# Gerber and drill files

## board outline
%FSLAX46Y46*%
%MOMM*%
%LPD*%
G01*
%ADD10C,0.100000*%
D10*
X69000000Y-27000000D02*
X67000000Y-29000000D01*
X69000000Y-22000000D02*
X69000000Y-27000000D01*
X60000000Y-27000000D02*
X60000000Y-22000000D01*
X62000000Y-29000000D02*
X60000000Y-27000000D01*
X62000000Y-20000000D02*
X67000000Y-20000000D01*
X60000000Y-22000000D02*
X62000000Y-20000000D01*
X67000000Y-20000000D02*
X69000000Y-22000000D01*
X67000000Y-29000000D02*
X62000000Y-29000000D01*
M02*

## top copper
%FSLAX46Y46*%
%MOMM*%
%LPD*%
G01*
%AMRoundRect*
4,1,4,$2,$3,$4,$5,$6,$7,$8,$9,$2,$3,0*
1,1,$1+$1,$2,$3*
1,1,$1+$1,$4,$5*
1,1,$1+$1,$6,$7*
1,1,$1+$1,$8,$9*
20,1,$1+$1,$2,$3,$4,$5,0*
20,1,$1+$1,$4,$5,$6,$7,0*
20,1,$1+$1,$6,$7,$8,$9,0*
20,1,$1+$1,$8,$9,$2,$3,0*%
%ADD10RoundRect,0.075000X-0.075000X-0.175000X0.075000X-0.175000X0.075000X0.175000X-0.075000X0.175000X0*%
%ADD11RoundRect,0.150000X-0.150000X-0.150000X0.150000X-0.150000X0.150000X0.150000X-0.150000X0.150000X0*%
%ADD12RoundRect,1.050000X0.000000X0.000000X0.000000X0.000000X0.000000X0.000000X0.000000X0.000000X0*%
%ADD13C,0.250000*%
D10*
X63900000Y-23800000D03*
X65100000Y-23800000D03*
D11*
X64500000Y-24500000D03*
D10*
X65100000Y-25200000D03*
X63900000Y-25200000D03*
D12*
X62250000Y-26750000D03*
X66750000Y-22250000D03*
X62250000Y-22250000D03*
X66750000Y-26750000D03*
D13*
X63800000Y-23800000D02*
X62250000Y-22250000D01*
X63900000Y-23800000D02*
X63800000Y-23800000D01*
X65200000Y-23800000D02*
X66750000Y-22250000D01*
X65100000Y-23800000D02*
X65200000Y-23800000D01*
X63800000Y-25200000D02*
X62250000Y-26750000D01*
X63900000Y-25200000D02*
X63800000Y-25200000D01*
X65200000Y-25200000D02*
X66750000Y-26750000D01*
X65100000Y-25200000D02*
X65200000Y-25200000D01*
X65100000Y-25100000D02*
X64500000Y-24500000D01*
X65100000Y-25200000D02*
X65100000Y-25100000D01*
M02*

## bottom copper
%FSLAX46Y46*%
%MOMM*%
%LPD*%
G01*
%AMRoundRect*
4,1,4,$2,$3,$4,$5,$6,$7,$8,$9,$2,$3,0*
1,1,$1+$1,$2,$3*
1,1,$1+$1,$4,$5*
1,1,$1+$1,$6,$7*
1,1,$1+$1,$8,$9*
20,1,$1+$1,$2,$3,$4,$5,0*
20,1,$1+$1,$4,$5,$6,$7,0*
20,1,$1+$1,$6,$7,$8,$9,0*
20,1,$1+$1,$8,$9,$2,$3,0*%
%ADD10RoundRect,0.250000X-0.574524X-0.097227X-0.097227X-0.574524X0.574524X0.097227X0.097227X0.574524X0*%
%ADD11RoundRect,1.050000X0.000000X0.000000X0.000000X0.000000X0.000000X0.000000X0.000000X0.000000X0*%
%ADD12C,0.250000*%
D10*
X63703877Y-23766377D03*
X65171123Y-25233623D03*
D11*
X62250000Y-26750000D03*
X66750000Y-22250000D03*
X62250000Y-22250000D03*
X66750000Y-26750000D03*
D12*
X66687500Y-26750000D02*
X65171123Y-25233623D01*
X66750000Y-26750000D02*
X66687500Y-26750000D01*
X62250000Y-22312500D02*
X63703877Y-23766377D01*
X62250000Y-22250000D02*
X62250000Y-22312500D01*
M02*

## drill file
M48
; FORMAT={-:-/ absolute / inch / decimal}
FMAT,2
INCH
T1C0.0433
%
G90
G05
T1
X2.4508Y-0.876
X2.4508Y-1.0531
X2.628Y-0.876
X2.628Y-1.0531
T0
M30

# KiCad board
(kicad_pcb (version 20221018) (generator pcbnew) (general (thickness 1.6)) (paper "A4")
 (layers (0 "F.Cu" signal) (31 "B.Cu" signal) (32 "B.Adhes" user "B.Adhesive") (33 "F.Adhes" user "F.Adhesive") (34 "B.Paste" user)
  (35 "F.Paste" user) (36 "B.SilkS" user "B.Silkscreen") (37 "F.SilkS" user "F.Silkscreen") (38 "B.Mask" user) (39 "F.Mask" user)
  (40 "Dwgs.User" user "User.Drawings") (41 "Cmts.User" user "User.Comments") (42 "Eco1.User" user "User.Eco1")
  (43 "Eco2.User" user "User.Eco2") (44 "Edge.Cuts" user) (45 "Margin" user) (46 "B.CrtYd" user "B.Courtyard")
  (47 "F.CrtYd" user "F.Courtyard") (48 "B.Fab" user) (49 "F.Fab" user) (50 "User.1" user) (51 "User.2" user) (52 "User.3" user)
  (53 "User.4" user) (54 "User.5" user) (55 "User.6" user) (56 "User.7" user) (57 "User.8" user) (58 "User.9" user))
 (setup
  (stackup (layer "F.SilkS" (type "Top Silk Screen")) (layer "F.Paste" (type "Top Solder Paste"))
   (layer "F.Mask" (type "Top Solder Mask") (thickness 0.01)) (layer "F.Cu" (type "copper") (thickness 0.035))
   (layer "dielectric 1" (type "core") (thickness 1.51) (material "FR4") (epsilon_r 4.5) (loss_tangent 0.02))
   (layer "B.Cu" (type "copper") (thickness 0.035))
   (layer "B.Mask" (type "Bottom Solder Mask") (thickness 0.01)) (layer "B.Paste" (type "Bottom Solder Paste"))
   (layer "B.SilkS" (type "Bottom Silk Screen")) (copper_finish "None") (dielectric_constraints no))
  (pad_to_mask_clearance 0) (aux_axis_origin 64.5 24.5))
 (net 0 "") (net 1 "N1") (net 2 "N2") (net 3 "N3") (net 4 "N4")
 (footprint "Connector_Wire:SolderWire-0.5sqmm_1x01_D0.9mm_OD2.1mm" (layer "F.Cu") (at 62.25 26.75)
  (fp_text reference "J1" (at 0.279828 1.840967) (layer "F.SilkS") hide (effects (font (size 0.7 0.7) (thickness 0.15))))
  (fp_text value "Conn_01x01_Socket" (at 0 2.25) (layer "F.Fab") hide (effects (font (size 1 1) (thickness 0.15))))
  (pad "1" thru_hole roundrect (at 0 0) (size 2.1 2.1) (drill 1.1) (layers "*.Cu" "*.Mask") (roundrect_rratio 0.5) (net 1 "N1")))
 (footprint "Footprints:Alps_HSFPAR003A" (layer "F.Cu") (at 64.5 24.5)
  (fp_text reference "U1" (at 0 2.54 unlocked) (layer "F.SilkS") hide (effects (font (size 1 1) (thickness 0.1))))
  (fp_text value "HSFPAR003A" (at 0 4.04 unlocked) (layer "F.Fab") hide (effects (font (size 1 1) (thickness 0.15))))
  (pad "1" smd roundrect (at -0.6 -0.7) (size 0.3 0.5) (layers "F.Cu" "F.Paste" "F.Mask") (roundrect_rratio 0.25) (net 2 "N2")
   (thermal_bridge_angle 45))
  (pad "2" smd roundrect (at 0.6 -0.7) (size 0.3 0.5) (layers "F.Cu" "F.Paste" "F.Mask") (roundrect_rratio 0.25) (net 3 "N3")
   (thermal_bridge_angle 45))
  (pad "3" smd roundrect (at 0 0) (size 0.6 0.6) (layers "F.Cu" "F.Paste" "F.Mask") (roundrect_rratio 0.25) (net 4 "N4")
   (thermal_bridge_angle 45))
  (pad "3" smd roundrect (at 0.6 0.7) (size 0.3 0.5) (layers "F.Cu" "F.Paste" "F.Mask") (roundrect_rratio 0.25) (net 4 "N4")
   (thermal_bridge_angle 45))
  (pad "4" smd roundrect (at -0.6 0.7) (size 0.3 0.5) (layers "F.Cu" "F.Paste" "F.Mask") (roundrect_rratio 0.25) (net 1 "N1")
   (thermal_bridge_angle 45)))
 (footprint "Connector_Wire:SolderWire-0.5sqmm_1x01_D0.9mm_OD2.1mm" (layer "F.Cu") (at 66.75 22.25)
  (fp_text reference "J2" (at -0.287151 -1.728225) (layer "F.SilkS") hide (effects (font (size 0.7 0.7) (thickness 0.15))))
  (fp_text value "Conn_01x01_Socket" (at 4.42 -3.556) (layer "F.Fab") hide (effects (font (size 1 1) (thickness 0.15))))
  (pad "1" thru_hole roundrect (at 0 0) (size 2.1 2.1) (drill 1.1) (layers "*.Cu" "*.Mask") (roundrect_rratio 0.5) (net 3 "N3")))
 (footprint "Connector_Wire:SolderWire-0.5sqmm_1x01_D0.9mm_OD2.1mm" (layer "F.Cu") (at 62.25 22.25)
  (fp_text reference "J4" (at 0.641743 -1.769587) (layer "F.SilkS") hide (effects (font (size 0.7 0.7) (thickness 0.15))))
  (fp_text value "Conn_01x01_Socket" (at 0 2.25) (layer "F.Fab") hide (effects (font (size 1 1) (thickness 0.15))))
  (pad "1" thru_hole roundrect (at 0 0) (size 2.1 2.1) (drill 1.1) (layers "*.Cu" "*.Mask") (roundrect_rratio 0.5) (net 2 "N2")))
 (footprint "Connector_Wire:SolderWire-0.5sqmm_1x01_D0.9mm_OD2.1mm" (layer "F.Cu") (at 66.75 26.75)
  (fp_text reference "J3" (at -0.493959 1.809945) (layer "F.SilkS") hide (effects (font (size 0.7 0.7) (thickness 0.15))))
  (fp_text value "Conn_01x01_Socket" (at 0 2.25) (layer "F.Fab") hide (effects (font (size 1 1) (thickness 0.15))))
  (pad "1" thru_hole roundrect (at 0 0) (size 2.1 2.1) (drill 1.1) (layers "*.Cu" "*.Mask") (roundrect_rratio 0.5) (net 4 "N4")
   (clearance -1)))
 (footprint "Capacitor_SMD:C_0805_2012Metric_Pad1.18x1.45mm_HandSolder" (layer "B.Cu") (at 64.4375 24.5 -45)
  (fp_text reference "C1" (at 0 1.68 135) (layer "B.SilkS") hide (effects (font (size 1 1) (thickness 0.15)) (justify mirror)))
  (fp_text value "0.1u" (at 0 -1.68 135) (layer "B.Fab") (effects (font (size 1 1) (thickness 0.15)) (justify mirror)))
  (pad "1" smd roundrect (at -1.0375 0 315) (size 1.175 1.45) (layers "B.Cu" "B.Paste" "B.Mask") (roundrect_rratio 0.2127659574)
   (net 2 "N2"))
  (pad "2" smd roundrect (at 1.0375 0 315) (size 1.175 1.45) (layers "B.Cu" "B.Paste" "B.Mask") (roundrect_rratio 0.2127659574) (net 4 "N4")))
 (gr_line (start 69 27) (end 67 29) (stroke (width 0.1) (type default)) (layer "Edge.Cuts"))
 (gr_line (start 69 22) (end 69 27) (stroke (width 0.1) (type default)) (layer "Edge.Cuts"))
 (gr_line (start 60 27) (end 60 22) (stroke (width 0.1) (type default)) (layer "Edge.Cuts"))
 (gr_line (start 62 29) (end 60 27) (stroke (width 0.1) (type default)) (layer "Edge.Cuts"))
 (gr_line (start 62 20) (end 67 20) (stroke (width 0.1) (type default)) (layer "Edge.Cuts"))
 (gr_line (start 60 22) (end 62 20) (stroke (width 0.1) (type default)) (layer "Edge.Cuts"))
 (gr_line (start 67 20) (end 69 22) (stroke (width 0.1) (type default)) (layer "Edge.Cuts"))
 (gr_line (start 67 29) (end 62 29) (stroke (width 0.1) (type default)) (layer "Edge.Cuts"))
 (segment (start 63.8 23.8) (end 62.25 22.25) (width 0.25) (layer "F.Cu") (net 2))
 (segment (start 63.9 23.8) (end 63.8 23.8) (width 0.25) (layer "F.Cu") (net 2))
 (segment (start 62.25 22.25) (end 62.25 22.3125) (width 0.25) (layer "B.Cu") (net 2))
 (segment (start 62.25 22.3125) (end 63.703877 23.766377) (width 0.25) (layer "B.Cu") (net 2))
 (segment (start 65.2 23.8) (end 66.75 22.25) (width 0.25) (layer "F.Cu") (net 3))
 (segment (start 65.1 23.8) (end 65.2 23.8) (width 0.25) (layer "F.Cu") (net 3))
 (segment (start 65.1 25.1) (end 64.5 24.5) (width 0.25) (layer "F.Cu") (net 4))
 (segment (start 65.1 25.2) (end 65.1 25.1) (width 0.25) (layer "F.Cu") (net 4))
 (segment (start 65.2 25.2) (end 66.75 26.75) (width 0.25) (layer "F.Cu") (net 4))
 (segment (start 65.1 25.2) (end 65.2 25.2) (width 0.25) (layer "F.Cu") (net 4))
 (segment (start 66.75 26.75) (end 66.6875 26.75) (width 0.25) (layer "B.Cu") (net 4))
 (segment (start 66.6875 26.75) (end 65.171123 25.233623) (width 0.25) (layer "B.Cu") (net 4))
 (segment (start 63.9 25.2) (end 63.8 25.2) (width 0.25) (layer "F.Cu") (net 1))
 (segment (start 63.8 25.2) (end 62.25 26.75) (width 0.25) (layer "F.Cu") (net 1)))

